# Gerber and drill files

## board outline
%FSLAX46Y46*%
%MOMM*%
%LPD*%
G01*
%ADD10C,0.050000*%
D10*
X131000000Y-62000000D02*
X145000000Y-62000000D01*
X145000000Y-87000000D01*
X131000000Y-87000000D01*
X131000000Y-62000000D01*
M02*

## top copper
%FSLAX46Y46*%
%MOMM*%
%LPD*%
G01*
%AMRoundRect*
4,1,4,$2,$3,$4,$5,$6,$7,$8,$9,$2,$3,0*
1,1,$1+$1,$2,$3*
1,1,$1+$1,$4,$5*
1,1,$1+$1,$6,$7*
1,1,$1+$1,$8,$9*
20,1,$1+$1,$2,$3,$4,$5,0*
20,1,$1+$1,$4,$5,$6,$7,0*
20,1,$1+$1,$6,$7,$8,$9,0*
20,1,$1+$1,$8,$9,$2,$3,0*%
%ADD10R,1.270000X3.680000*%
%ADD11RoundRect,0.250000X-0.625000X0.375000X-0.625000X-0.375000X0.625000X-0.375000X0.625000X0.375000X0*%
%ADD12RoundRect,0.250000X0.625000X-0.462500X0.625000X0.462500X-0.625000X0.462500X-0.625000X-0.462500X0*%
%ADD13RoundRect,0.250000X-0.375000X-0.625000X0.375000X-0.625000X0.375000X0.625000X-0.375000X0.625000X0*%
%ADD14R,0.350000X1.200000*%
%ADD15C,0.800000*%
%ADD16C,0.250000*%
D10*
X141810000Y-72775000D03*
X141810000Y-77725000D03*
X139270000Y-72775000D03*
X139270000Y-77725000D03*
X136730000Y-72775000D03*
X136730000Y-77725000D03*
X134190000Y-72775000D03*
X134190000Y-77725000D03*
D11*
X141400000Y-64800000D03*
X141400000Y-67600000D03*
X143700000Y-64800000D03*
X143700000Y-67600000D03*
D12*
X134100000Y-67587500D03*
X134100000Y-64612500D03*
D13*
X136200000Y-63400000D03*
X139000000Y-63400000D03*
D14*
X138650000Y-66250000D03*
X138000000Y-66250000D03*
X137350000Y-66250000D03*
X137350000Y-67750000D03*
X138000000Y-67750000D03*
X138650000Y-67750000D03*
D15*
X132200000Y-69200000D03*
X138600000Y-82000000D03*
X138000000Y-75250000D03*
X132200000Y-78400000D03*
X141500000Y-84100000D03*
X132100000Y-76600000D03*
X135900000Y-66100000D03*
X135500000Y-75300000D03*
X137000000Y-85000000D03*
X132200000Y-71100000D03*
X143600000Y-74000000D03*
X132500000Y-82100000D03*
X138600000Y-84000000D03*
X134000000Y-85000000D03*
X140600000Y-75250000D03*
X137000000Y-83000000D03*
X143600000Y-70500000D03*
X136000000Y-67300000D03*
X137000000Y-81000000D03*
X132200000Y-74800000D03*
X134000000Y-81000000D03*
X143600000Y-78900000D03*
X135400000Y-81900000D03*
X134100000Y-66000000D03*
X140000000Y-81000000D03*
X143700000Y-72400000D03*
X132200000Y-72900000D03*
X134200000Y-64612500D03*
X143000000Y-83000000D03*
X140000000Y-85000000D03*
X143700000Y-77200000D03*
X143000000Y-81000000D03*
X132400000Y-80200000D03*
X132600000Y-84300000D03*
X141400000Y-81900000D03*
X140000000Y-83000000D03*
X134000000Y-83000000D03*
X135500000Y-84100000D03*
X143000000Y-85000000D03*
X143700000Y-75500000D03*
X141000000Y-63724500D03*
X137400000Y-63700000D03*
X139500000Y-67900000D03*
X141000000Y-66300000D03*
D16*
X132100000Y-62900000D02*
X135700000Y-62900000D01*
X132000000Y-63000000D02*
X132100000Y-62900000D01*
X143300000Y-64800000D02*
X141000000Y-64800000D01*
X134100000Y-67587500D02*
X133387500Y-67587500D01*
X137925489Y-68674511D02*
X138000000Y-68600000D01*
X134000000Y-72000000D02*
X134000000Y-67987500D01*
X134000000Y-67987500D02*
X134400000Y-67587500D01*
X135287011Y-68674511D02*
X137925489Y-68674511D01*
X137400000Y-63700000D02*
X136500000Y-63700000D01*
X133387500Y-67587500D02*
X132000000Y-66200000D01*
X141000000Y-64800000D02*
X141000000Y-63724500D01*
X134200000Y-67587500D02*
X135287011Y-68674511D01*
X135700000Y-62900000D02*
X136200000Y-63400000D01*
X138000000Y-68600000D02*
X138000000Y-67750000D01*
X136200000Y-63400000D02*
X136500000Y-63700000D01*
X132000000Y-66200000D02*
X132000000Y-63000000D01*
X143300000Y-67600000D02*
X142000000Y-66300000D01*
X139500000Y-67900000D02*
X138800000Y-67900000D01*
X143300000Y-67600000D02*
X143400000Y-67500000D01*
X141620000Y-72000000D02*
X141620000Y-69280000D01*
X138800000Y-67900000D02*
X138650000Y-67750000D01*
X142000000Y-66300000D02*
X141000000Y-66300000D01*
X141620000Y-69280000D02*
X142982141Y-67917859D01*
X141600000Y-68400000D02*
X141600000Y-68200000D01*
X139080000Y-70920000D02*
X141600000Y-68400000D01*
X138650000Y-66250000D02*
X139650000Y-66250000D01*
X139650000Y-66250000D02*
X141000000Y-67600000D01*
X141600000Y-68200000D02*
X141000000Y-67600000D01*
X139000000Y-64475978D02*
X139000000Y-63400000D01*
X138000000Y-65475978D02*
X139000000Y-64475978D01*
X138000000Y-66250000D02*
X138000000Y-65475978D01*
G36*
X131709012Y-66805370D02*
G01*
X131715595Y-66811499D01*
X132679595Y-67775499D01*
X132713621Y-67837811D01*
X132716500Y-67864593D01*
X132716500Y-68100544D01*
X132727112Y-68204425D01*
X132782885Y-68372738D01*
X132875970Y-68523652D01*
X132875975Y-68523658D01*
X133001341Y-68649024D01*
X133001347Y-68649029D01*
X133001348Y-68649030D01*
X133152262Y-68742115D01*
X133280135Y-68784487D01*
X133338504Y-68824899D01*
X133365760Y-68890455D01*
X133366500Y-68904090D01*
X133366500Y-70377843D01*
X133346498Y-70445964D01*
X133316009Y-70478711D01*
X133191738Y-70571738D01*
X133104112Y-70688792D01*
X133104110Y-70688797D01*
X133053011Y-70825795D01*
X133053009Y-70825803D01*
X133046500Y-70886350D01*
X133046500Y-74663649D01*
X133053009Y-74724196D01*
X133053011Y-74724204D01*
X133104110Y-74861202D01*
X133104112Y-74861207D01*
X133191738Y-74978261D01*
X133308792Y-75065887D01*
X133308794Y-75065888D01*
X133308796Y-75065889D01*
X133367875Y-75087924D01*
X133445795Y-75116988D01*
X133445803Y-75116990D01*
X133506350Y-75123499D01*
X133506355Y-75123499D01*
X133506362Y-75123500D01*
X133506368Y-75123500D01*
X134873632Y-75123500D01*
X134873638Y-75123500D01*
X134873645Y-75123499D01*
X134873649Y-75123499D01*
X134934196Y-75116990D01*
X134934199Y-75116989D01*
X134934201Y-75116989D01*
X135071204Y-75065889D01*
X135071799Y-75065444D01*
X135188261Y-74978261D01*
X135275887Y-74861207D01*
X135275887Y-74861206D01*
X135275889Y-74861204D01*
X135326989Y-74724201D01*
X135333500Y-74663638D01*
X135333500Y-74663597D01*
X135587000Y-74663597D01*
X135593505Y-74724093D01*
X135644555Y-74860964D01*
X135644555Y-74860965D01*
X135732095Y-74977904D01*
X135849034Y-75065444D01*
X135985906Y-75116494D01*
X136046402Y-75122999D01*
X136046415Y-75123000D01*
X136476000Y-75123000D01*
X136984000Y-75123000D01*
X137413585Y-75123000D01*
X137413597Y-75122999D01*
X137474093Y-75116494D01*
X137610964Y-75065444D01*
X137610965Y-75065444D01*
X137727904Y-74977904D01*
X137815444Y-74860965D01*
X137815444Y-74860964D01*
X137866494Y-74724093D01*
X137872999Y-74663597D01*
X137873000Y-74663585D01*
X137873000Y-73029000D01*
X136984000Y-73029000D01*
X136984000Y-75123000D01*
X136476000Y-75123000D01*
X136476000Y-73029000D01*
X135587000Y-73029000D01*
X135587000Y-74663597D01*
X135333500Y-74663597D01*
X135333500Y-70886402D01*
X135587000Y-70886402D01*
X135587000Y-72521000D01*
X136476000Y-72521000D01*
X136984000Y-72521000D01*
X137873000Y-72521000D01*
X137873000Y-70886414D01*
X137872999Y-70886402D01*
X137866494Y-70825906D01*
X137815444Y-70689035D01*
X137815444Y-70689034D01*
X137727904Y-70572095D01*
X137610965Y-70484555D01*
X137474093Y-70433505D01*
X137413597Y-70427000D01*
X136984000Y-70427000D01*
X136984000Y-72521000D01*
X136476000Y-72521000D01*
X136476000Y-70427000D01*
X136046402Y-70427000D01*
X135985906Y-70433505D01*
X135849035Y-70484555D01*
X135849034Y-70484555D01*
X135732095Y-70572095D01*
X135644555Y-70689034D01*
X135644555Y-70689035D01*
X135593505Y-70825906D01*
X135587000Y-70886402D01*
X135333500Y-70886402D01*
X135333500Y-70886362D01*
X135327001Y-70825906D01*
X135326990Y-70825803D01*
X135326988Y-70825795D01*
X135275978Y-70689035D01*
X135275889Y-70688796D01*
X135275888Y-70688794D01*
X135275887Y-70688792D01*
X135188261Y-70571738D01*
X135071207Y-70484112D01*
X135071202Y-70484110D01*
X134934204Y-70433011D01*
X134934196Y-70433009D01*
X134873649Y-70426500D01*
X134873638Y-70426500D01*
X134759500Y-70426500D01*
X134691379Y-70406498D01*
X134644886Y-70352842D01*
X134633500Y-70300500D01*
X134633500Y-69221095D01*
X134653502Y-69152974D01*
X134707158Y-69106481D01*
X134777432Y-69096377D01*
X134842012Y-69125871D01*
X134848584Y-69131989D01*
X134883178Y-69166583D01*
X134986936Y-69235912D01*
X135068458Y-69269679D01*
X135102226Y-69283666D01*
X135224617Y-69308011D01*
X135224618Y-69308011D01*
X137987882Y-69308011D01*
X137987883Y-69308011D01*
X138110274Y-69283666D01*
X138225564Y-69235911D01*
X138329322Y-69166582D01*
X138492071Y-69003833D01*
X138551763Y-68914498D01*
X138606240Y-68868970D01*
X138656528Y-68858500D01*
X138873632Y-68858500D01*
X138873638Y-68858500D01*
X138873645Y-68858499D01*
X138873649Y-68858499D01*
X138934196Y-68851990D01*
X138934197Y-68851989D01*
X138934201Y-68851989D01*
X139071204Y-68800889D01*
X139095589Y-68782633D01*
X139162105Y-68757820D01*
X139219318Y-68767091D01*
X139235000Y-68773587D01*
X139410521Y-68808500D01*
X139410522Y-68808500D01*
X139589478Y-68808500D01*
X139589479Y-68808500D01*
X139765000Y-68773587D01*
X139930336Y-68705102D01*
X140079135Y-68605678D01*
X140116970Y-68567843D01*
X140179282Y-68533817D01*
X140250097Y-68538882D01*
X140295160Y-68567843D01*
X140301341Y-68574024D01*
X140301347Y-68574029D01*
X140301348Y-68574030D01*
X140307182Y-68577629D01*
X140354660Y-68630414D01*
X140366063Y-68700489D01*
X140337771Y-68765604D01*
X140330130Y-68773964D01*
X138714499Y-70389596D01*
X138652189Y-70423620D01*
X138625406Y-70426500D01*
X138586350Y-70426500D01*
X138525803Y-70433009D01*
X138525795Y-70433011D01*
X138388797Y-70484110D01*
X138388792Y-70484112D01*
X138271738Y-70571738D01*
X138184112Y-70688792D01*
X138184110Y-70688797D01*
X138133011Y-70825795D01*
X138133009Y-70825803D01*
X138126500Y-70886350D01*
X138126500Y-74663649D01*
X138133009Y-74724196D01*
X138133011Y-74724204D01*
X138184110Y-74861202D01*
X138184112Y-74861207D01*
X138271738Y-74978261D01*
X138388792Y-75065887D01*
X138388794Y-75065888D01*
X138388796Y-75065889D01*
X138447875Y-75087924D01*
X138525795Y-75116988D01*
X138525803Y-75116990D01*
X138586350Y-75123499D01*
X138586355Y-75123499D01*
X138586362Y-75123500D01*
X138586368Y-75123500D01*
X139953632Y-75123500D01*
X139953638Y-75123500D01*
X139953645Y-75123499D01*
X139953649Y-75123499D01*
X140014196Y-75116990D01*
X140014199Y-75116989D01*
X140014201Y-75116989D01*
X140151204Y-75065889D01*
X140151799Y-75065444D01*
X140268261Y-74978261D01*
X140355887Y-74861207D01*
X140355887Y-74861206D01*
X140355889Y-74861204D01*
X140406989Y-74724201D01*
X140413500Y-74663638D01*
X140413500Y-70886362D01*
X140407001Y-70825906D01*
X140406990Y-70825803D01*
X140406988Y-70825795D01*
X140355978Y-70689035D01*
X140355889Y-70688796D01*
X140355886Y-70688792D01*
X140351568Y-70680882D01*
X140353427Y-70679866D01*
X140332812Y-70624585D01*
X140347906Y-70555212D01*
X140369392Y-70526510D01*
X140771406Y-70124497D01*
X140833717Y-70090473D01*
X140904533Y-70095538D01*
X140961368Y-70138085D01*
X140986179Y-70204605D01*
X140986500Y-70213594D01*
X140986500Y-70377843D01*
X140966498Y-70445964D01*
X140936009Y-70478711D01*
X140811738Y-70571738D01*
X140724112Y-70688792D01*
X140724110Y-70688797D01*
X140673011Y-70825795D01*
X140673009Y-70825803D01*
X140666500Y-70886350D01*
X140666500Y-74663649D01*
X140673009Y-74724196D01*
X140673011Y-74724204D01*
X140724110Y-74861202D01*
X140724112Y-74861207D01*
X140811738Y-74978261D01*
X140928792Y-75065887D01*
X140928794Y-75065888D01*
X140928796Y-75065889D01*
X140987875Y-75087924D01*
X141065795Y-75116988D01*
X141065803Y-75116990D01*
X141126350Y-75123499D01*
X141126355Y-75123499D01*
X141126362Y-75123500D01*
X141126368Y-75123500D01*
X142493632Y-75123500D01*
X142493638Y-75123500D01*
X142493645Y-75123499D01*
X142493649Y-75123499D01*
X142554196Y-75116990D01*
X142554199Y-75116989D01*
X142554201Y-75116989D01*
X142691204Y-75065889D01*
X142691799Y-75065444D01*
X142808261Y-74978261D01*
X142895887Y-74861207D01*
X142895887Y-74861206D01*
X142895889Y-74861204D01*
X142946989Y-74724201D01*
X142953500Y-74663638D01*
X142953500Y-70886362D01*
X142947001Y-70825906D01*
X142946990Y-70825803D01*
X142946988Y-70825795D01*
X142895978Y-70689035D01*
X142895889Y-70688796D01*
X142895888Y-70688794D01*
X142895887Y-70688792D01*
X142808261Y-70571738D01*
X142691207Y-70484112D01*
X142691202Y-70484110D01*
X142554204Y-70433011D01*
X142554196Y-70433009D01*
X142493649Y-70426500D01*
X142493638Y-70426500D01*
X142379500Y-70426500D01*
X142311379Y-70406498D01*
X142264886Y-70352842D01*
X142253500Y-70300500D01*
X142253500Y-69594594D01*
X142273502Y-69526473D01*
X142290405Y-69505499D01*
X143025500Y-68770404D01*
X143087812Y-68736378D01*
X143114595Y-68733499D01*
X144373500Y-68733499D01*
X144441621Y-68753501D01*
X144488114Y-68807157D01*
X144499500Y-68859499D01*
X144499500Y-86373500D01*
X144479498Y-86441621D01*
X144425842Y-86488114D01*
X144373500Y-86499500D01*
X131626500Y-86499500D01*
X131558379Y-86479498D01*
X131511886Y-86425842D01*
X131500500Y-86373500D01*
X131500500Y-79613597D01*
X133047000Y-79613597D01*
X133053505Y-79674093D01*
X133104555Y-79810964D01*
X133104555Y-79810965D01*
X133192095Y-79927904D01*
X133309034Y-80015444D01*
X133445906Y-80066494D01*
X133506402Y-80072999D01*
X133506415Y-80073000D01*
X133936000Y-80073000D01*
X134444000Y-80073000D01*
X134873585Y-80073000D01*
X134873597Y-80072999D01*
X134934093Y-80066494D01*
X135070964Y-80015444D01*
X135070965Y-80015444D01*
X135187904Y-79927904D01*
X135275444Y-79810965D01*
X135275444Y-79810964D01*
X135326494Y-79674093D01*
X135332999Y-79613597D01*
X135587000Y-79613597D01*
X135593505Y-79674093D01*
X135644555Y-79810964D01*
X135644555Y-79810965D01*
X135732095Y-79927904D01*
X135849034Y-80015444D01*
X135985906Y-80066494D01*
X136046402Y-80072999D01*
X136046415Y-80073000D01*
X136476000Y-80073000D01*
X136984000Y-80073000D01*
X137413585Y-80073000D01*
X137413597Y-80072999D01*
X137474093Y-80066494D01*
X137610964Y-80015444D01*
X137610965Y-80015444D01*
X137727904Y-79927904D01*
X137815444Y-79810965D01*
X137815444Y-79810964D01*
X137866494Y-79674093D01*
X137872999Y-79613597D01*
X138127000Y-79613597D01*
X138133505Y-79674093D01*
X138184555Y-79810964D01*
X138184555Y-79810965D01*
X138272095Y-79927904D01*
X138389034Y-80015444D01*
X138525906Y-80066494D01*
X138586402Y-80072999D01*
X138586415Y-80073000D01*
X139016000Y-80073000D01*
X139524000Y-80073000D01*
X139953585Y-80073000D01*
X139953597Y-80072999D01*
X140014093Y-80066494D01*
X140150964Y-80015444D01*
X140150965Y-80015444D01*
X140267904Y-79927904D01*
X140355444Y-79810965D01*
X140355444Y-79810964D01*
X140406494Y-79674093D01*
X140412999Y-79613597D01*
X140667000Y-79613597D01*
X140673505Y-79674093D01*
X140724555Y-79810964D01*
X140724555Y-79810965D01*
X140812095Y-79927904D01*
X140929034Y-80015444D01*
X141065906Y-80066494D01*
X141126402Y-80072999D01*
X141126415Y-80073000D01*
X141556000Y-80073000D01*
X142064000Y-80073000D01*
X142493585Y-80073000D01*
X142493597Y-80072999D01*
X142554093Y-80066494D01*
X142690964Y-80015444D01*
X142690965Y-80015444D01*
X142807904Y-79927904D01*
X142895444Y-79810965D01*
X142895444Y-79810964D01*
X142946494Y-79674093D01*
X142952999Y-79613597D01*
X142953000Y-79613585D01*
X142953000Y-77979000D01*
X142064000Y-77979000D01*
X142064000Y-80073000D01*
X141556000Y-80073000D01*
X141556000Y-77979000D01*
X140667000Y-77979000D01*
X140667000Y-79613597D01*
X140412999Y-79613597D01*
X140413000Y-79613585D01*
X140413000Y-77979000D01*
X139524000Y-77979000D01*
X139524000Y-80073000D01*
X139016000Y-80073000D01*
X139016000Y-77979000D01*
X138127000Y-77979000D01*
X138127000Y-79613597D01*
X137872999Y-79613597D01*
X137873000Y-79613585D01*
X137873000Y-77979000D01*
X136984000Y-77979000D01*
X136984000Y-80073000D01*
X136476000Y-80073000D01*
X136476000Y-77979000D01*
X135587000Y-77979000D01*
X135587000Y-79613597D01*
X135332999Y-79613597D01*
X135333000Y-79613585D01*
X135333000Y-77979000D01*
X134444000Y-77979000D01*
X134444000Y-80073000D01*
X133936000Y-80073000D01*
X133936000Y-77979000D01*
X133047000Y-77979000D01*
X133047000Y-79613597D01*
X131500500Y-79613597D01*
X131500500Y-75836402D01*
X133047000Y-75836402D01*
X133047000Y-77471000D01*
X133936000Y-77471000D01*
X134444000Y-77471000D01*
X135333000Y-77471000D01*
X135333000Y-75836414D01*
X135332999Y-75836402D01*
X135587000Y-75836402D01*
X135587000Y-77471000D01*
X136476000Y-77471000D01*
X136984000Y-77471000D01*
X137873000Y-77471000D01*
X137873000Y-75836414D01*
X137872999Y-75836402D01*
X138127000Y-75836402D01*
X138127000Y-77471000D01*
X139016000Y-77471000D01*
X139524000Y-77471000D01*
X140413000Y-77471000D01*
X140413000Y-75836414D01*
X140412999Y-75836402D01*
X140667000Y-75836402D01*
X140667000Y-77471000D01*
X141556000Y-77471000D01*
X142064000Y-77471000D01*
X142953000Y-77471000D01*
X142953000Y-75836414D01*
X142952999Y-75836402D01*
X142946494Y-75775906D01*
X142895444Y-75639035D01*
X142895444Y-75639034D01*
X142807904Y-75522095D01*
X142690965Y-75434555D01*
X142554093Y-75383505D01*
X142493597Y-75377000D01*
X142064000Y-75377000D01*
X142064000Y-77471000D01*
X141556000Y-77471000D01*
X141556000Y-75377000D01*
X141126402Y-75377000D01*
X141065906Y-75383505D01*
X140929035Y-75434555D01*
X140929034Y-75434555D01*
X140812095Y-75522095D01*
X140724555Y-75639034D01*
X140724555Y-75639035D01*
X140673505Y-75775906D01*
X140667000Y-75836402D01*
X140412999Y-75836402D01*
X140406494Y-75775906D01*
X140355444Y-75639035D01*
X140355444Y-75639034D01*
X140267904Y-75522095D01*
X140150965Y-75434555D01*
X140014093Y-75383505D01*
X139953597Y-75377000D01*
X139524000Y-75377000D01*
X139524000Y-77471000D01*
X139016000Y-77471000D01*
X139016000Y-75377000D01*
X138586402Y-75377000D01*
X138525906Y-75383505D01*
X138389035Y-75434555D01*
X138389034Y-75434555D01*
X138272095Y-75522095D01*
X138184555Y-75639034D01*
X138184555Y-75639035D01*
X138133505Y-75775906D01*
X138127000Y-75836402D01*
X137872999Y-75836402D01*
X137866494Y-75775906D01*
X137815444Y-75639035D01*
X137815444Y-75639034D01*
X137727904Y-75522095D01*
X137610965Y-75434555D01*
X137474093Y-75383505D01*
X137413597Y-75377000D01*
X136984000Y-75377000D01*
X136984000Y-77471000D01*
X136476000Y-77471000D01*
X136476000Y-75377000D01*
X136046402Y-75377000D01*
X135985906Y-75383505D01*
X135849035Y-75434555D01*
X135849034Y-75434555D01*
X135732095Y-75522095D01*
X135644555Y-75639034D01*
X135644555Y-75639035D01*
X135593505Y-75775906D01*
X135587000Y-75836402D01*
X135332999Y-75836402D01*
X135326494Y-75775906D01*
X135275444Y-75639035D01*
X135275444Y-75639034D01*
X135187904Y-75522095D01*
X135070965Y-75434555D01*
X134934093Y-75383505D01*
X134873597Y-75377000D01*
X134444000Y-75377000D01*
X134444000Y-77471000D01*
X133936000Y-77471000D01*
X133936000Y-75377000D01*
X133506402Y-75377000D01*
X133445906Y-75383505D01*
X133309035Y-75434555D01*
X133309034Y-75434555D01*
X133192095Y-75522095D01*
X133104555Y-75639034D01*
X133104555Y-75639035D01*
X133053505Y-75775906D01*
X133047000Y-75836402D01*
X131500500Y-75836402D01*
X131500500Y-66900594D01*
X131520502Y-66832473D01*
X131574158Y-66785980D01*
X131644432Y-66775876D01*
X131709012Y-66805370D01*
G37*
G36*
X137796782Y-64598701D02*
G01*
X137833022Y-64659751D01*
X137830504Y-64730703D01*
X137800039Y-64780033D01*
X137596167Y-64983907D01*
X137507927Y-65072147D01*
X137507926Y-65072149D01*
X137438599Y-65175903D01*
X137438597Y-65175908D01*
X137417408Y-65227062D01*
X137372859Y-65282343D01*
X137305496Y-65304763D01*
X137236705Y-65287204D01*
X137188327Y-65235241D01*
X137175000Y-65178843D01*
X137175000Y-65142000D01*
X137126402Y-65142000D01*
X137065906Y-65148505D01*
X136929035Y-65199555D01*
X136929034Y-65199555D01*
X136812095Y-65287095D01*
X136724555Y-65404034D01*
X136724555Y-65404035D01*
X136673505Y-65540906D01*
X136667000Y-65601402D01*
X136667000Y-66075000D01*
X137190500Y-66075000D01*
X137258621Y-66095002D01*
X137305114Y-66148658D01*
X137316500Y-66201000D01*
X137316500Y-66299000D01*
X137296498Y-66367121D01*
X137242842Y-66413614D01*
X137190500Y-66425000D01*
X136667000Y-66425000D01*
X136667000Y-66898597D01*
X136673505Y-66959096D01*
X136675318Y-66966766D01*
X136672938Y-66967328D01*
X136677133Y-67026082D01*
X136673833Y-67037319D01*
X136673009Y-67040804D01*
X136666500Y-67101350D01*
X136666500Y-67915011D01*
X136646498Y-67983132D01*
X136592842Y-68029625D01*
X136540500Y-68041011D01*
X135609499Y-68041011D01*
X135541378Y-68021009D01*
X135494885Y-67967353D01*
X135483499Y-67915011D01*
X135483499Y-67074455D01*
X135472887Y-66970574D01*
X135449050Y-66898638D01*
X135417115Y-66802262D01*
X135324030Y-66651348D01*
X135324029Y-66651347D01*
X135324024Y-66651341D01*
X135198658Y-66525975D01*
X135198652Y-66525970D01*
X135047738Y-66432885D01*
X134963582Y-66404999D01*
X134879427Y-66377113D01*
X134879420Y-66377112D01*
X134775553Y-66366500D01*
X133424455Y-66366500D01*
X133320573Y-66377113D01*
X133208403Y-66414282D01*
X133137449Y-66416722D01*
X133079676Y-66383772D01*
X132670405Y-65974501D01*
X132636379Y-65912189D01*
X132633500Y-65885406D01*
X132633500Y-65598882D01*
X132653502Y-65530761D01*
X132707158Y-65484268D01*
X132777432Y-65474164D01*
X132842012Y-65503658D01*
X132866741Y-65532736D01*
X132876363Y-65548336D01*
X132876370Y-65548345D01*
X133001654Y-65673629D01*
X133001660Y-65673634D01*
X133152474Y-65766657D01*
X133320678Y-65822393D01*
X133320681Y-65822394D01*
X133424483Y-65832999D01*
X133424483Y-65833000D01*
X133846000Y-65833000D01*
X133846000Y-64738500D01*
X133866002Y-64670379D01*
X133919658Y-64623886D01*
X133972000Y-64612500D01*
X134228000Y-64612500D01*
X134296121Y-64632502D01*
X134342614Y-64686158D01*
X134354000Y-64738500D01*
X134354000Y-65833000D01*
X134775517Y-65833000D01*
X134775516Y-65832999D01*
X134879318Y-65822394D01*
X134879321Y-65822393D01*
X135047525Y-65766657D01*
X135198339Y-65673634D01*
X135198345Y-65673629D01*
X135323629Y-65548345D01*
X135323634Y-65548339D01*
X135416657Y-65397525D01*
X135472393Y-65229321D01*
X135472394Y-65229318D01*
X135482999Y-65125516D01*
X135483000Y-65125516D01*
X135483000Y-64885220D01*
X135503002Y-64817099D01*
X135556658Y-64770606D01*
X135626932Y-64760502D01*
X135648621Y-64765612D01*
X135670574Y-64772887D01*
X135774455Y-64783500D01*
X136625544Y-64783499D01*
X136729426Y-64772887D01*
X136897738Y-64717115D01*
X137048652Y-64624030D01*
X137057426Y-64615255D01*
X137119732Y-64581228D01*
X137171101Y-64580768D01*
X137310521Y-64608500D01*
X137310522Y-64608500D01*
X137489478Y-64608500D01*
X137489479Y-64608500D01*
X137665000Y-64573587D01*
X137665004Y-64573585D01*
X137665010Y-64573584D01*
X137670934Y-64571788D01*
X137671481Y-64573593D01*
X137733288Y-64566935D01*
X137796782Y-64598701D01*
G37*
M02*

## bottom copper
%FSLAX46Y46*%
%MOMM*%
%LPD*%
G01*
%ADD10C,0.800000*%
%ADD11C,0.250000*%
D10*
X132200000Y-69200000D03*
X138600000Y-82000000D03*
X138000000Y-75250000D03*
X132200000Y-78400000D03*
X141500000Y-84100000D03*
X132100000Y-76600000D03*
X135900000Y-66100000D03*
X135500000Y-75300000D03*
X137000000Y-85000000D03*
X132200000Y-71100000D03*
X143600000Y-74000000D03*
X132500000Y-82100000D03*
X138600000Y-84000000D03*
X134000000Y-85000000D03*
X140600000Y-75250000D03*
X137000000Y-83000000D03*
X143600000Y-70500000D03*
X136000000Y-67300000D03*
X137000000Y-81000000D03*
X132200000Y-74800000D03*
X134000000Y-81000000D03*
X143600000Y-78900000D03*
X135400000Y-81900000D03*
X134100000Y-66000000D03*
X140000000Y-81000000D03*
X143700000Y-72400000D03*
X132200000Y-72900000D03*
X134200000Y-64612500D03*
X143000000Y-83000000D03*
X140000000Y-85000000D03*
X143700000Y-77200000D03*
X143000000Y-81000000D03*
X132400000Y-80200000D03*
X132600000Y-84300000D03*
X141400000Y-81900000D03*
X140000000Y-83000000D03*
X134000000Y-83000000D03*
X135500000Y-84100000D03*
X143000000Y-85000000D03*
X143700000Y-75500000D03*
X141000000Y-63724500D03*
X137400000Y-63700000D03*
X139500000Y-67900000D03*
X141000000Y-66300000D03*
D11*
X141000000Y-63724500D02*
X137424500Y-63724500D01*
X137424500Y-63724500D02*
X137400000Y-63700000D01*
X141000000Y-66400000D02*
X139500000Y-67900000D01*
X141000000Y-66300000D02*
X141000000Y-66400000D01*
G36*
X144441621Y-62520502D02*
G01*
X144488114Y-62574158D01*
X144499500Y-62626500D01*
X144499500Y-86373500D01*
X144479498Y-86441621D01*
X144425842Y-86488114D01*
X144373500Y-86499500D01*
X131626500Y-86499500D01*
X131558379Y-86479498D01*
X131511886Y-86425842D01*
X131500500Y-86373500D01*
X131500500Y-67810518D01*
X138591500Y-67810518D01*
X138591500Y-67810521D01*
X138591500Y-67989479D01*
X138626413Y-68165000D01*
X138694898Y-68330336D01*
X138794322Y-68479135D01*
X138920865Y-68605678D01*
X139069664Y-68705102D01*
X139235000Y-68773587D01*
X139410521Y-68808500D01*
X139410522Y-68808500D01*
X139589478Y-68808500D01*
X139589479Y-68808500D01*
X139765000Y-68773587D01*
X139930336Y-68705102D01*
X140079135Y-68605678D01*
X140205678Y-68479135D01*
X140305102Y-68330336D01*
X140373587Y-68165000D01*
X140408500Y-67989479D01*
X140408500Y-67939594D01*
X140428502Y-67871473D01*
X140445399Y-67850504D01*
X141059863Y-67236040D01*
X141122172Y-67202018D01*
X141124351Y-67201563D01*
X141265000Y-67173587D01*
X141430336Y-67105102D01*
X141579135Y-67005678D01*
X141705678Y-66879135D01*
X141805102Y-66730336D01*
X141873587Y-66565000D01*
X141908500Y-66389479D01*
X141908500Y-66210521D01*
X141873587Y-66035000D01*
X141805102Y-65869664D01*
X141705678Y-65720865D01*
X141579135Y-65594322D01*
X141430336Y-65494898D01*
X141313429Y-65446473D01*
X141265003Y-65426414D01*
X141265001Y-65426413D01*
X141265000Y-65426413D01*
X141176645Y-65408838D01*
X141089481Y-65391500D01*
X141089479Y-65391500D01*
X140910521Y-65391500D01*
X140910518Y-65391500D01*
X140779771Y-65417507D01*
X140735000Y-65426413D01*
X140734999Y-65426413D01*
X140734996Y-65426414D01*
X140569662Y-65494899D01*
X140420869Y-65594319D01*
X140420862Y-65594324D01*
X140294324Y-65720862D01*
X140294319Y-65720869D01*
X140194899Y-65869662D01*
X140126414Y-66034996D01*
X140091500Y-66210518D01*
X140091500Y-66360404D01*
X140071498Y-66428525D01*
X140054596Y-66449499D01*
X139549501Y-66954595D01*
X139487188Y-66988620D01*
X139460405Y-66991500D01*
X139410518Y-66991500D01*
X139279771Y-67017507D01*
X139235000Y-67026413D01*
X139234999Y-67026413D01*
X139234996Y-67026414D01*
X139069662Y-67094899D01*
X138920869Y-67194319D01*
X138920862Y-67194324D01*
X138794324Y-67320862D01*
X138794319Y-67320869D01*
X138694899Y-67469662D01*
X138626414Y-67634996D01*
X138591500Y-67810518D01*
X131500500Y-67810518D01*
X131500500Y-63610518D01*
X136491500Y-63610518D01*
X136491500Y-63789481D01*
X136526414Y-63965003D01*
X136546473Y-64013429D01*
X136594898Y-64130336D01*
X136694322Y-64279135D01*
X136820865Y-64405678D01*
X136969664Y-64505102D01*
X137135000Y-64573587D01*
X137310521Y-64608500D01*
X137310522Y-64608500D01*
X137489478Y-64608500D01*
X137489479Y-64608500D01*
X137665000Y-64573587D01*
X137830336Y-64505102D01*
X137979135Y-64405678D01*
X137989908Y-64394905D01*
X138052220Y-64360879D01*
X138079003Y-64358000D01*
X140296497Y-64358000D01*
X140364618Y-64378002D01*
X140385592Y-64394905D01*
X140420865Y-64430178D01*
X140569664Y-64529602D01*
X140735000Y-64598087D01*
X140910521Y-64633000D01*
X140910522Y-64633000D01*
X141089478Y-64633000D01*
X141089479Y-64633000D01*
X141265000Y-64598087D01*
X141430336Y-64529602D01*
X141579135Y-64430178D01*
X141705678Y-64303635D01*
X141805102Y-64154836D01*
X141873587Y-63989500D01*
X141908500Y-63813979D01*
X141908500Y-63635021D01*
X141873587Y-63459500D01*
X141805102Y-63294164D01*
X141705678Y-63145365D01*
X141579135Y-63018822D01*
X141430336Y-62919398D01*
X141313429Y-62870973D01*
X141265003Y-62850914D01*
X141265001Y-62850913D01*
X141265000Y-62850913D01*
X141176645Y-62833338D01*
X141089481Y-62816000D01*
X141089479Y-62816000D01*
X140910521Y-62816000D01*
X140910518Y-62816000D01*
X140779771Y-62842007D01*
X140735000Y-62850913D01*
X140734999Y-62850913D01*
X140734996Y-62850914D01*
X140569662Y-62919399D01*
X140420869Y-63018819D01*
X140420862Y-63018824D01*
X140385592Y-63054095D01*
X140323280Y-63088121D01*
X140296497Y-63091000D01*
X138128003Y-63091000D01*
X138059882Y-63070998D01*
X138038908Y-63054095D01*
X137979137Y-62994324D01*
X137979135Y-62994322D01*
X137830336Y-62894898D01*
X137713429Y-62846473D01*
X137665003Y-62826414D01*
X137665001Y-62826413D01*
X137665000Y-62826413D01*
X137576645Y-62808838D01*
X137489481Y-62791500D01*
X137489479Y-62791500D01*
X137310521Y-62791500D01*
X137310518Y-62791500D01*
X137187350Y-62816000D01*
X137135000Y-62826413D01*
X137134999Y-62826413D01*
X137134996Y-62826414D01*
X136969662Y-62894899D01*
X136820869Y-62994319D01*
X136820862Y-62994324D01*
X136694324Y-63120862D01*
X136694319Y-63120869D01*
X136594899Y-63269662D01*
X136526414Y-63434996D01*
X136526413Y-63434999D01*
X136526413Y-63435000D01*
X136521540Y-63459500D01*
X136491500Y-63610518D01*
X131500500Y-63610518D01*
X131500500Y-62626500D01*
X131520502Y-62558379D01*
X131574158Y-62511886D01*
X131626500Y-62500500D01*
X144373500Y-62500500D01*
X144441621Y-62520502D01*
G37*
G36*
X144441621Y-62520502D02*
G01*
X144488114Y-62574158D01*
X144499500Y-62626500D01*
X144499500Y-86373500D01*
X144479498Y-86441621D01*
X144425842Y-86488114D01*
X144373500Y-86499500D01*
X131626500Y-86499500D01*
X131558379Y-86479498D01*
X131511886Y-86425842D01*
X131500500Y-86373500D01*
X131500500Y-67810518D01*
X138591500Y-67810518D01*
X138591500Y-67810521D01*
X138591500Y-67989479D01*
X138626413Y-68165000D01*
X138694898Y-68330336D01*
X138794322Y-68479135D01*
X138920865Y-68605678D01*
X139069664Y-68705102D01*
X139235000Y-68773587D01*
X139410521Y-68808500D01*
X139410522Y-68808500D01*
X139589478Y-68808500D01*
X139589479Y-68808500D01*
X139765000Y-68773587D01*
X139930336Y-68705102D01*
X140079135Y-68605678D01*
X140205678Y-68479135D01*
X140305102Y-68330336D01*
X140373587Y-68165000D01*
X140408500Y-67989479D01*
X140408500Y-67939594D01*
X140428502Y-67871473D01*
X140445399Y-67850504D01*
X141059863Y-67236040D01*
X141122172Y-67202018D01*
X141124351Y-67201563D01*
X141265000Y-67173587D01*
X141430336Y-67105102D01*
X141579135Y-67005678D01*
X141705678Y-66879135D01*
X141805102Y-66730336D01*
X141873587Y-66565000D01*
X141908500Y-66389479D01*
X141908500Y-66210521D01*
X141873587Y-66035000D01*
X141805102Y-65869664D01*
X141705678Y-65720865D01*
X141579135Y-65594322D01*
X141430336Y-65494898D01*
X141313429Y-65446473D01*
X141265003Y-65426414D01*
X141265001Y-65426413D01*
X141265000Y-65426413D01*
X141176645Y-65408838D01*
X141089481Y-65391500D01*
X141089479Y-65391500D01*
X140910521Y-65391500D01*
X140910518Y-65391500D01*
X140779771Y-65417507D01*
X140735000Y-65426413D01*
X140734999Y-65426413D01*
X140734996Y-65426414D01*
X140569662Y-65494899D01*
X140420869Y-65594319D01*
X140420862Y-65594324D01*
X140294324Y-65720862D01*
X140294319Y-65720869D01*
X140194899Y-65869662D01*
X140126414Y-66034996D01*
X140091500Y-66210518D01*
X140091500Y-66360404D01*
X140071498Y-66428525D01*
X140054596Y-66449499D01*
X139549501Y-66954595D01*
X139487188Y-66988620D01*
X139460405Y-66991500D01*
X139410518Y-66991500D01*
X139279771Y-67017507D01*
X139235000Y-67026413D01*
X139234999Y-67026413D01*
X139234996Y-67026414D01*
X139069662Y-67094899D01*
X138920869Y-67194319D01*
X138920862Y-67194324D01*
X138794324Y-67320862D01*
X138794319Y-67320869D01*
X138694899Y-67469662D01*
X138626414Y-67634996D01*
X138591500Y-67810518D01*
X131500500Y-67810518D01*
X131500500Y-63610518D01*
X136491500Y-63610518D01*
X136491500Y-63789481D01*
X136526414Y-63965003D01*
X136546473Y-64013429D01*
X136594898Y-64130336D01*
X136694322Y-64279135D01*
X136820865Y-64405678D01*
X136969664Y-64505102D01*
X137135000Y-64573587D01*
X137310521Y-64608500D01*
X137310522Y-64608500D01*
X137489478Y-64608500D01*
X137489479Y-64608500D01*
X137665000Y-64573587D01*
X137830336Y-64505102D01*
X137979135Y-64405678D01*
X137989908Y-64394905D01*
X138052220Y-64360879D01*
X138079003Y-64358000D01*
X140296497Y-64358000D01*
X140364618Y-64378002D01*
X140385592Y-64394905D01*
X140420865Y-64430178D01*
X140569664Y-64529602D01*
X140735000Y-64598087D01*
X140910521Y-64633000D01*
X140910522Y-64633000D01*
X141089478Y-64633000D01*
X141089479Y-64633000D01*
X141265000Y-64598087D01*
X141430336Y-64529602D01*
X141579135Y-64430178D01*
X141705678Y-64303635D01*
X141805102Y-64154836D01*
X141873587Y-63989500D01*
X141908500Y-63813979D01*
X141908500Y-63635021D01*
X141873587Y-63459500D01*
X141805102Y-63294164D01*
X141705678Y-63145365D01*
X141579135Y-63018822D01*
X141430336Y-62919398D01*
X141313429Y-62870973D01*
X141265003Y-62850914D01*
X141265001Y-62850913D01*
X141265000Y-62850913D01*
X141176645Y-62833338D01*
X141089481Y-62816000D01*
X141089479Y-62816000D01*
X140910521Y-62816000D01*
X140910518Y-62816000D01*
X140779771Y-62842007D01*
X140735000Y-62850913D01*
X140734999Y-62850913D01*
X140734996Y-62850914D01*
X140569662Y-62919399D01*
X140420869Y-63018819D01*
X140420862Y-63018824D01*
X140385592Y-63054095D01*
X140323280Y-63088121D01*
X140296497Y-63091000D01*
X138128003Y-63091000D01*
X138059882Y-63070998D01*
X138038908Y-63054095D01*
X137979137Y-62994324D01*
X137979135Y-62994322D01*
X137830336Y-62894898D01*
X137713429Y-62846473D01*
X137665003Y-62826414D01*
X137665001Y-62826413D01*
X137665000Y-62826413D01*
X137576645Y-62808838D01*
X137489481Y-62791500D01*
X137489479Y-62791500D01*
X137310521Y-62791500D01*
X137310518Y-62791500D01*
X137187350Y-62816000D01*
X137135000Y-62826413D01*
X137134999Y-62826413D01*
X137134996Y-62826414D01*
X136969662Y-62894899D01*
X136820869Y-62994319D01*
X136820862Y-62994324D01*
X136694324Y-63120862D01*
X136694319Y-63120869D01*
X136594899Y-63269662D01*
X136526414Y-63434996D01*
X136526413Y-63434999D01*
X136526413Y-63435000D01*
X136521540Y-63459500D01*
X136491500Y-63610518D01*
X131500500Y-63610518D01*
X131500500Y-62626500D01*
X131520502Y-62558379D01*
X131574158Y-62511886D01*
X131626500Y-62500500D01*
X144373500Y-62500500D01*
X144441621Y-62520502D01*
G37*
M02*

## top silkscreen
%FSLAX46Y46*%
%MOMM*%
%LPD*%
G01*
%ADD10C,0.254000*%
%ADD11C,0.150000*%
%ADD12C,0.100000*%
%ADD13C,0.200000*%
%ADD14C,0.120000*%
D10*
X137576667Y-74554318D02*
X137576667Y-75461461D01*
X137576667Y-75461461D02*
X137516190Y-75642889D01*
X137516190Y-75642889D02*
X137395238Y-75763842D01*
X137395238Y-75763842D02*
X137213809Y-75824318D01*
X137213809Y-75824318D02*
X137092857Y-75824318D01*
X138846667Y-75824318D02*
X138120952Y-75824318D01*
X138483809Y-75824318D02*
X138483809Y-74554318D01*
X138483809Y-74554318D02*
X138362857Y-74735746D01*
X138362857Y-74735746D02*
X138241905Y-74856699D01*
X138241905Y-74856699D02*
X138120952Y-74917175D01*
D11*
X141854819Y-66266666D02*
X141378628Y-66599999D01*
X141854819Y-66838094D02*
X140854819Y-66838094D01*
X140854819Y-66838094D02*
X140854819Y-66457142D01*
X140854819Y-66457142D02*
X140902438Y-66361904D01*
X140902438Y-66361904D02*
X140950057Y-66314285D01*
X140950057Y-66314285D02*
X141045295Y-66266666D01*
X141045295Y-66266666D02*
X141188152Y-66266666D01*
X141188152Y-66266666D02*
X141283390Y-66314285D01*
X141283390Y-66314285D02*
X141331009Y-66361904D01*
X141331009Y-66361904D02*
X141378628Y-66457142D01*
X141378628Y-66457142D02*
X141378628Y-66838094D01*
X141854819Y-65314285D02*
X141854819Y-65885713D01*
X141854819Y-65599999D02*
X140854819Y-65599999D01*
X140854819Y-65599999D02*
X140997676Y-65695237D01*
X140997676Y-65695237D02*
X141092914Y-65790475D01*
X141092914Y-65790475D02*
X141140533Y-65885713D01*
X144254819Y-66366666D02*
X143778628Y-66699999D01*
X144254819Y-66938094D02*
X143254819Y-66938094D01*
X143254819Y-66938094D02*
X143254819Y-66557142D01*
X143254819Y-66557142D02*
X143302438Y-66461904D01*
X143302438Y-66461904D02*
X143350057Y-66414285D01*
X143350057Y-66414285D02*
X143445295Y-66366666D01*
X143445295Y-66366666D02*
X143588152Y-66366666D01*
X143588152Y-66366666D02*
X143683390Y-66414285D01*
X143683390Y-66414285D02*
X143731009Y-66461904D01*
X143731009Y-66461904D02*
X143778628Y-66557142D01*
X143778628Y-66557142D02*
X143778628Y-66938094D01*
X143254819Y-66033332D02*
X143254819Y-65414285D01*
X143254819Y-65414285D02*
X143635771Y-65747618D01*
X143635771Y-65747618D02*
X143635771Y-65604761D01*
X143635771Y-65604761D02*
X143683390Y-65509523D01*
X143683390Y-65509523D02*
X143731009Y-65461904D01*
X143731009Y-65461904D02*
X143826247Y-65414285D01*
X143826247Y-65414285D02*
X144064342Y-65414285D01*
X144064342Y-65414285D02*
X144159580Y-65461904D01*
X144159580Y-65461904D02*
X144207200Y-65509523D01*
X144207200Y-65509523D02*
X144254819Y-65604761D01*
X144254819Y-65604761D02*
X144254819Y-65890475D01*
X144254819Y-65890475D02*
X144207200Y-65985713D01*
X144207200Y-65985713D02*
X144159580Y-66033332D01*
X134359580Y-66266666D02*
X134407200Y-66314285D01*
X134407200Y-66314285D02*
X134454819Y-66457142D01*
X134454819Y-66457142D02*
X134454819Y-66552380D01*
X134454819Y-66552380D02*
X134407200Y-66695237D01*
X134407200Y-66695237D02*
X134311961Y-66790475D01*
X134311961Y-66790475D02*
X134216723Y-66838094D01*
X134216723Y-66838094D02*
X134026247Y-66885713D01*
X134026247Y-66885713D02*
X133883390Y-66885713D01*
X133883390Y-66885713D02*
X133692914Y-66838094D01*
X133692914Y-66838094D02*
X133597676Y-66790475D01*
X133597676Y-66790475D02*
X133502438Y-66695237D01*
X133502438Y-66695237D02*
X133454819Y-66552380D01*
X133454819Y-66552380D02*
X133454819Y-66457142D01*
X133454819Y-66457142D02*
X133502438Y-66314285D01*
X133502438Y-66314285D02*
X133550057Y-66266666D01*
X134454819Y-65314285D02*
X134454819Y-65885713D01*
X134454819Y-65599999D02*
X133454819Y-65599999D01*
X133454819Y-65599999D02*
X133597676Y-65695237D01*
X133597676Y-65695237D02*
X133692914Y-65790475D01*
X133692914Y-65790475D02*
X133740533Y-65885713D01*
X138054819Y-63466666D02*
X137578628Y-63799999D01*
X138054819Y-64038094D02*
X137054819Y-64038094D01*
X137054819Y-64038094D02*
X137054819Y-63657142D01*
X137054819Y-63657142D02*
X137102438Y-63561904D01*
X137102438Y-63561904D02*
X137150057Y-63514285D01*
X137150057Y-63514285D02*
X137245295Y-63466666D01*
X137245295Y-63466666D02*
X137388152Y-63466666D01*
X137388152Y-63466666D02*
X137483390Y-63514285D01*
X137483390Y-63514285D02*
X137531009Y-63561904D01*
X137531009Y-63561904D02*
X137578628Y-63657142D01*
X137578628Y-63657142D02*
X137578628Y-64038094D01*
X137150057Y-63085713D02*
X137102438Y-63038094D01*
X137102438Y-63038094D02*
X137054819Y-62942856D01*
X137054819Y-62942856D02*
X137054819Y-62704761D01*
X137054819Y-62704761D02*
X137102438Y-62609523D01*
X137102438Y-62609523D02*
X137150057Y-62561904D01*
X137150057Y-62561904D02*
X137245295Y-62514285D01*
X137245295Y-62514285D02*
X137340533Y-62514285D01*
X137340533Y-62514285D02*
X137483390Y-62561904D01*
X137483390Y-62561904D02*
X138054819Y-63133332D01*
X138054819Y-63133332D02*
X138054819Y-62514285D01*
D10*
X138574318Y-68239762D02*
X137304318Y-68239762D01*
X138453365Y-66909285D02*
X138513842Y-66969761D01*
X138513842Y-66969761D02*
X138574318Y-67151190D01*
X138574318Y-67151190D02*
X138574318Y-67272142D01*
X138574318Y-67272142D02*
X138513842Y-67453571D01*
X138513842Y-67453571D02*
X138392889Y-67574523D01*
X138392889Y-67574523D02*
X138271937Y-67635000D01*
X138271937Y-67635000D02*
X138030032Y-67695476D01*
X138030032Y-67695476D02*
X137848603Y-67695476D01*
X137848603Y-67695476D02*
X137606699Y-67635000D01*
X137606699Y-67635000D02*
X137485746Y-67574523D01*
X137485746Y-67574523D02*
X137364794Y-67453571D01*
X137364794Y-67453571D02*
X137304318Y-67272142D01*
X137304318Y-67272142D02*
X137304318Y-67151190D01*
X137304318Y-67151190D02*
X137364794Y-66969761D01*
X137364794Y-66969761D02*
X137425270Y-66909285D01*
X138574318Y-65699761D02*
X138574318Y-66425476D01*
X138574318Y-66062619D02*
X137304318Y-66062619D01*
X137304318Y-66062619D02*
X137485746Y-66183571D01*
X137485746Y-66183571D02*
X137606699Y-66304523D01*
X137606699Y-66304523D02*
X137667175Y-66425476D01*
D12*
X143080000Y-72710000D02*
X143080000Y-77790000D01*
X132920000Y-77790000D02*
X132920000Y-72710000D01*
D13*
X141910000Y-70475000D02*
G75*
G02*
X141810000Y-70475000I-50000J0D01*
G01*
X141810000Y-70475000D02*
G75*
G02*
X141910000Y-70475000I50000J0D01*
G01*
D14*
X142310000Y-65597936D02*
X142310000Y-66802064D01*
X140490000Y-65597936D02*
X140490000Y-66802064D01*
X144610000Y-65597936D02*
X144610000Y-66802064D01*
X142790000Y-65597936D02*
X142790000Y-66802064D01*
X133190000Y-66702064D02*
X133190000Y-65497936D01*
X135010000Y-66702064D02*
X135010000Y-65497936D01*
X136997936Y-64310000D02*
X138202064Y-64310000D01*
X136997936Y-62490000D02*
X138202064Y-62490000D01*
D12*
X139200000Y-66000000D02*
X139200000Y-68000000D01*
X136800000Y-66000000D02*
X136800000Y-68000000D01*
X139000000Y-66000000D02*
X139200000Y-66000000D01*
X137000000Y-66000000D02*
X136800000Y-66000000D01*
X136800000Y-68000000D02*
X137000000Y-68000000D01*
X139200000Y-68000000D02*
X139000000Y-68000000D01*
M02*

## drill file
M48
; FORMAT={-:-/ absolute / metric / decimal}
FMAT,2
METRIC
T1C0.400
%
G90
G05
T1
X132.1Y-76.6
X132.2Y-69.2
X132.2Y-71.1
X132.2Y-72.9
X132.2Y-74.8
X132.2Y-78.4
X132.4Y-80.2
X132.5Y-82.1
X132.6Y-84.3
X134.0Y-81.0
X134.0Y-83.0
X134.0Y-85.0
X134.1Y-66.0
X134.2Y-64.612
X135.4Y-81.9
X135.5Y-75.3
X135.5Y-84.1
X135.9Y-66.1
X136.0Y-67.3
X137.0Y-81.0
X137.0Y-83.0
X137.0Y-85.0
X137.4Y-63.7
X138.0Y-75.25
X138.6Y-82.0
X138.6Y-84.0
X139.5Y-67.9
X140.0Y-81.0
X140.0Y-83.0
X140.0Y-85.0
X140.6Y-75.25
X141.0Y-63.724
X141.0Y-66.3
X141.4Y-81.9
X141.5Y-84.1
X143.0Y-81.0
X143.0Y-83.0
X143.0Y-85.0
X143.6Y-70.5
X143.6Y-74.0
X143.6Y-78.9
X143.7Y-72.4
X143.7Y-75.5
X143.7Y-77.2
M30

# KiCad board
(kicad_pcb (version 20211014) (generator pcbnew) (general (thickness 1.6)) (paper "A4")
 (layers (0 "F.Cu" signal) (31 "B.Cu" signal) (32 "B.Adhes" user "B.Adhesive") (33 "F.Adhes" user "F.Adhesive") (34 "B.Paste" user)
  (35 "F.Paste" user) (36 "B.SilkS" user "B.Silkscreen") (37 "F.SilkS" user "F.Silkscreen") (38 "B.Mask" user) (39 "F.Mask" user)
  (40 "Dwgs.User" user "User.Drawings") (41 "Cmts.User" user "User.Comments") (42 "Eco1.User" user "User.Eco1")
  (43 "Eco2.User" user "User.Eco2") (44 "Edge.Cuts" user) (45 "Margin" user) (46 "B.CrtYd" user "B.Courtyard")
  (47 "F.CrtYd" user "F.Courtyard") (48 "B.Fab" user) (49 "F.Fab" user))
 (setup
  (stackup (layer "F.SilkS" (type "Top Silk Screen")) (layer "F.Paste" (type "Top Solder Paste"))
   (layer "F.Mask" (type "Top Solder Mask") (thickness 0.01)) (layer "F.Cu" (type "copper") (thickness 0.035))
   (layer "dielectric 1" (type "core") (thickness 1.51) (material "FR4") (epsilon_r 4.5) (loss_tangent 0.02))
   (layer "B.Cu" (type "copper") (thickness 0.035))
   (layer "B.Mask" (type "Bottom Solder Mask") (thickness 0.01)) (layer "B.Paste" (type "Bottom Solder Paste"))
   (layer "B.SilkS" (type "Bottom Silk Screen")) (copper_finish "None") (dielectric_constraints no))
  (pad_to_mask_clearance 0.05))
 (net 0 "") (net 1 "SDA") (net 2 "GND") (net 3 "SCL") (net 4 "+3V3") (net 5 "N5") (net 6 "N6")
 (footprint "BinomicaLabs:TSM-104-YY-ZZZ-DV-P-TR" (layer "F.Cu") (at 138 75.25)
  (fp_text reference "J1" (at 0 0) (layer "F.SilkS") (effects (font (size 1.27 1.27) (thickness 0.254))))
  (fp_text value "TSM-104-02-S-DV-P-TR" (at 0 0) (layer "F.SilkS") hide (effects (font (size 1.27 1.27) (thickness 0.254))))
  (fp_line (start 5.08 -2.54) (end 5.08 2.54) (layer "F.SilkS") (width 0.1))
  (fp_line (start -5.08 2.54) (end -5.08 -2.54) (layer "F.SilkS") (width 0.1))
  (fp_circle (center 3.86 -4.775) (end 3.86 -4.725) (layer "F.SilkS") (width 0.2) (fill none))
  (pad "1" smd rect locked (at 3.81 -2.475) (size 1.27 3.68) (layers "F.Cu" "F.Paste" "F.Mask") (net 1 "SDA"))
  (pad "2" smd rect locked (at 3.81 2.475) (size 1.27 3.68) (layers "F.Cu" "F.Paste" "F.Mask") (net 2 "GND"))
  (pad "3" smd rect locked (at 1.27 -2.475) (size 1.27 3.68) (layers "F.Cu" "F.Paste" "F.Mask") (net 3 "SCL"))
  (pad "4" smd rect locked (at 1.27 2.475) (size 1.27 3.68) (layers "F.Cu" "F.Paste" "F.Mask") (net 2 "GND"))
  (pad "5" smd rect locked (at -1.27 -2.475) (size 1.27 3.68) (layers "F.Cu" "F.Paste" "F.Mask") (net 2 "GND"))
  (pad "6" smd rect locked (at -1.27 2.475) (size 1.27 3.68) (layers "F.Cu" "F.Paste" "F.Mask") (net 2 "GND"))
  (pad "7" smd rect locked (at -3.81 -2.475) (size 1.27 3.68) (layers "F.Cu" "F.Paste" "F.Mask") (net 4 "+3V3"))
  (pad "8" smd rect locked (at -3.81 2.475) (size 1.27 3.68) (layers "F.Cu" "F.Paste" "F.Mask") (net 2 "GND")))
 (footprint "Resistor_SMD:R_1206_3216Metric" (layer "F.Cu") (at 141.4 66.2 -90)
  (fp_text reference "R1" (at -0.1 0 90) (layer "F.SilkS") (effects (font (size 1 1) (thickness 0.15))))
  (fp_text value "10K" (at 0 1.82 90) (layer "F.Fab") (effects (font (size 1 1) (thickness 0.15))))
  (fp_line (start -0.602064 -0.91) (end 0.602064 -0.91) (layer "F.SilkS") (width 0.12))
  (fp_line (start -0.602064 0.91) (end 0.602064 0.91) (layer "F.SilkS") (width 0.12))
  (pad "1" smd roundrect locked (at -1.4 0 270) (size 1.25 1.75) (layers "F.Cu" "F.Paste" "F.Mask") (roundrect_rratio 0.2) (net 4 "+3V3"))
  (pad "2" smd roundrect locked (at 1.4 0 270) (size 1.25 1.75) (layers "F.Cu" "F.Paste" "F.Mask") (roundrect_rratio 0.2) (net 3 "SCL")))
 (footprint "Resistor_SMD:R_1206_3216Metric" (layer "F.Cu") (at 143.7 66.2 -90)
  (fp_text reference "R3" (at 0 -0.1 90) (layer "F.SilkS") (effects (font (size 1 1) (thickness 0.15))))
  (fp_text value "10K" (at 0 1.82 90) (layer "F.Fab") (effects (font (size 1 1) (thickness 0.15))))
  (fp_line (start -0.602064 -0.91) (end 0.602064 -0.91) (layer "F.SilkS") (width 0.12))
  (fp_line (start -0.602064 0.91) (end 0.602064 0.91) (layer "F.SilkS") (width 0.12))
  (pad "1" smd roundrect locked (at -1.4 0 270) (size 1.25 1.75) (layers "F.Cu" "F.Paste" "F.Mask") (roundrect_rratio 0.2) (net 4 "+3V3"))
  (pad "2" smd roundrect locked (at 1.4 0 270) (size 1.25 1.75) (layers "F.Cu" "F.Paste" "F.Mask") (roundrect_rratio 0.2) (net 1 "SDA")))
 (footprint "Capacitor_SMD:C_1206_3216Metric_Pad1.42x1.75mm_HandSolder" (layer "F.Cu") (at 134.1 66.1 90)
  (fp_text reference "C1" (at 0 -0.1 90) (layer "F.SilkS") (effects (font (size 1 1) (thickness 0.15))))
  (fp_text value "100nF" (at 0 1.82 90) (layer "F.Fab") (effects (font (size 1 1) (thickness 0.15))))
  (fp_line (start -0.602064 -0.91) (end 0.602064 -0.91) (layer "F.SilkS") (width 0.12))
  (fp_line (start -0.602064 0.91) (end 0.602064 0.91) (layer "F.SilkS") (width 0.12))
  (pad "1" smd roundrect locked (at -1.4875 0 90) (size 1.425 1.75) (layers "F.Cu" "F.Paste" "F.Mask") (roundrect_rratio 0.1754385965)
   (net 4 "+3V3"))
  (pad "2" smd roundrect locked (at 1.4875 0 90) (size 1.425 1.75) (layers "F.Cu" "F.Paste" "F.Mask") (roundrect_rratio 0.1754385965)
   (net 2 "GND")))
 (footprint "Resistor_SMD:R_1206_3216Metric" (layer "F.Cu") (at 137.6 63.4)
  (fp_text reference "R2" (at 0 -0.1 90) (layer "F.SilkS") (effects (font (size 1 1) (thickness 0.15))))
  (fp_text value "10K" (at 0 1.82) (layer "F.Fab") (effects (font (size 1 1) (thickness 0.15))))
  (fp_line (start -0.602064 0.91) (end 0.602064 0.91) (layer "F.SilkS") (width 0.12))
  (fp_line (start -0.602064 -0.91) (end 0.602064 -0.91) (layer "F.SilkS") (width 0.12))
  (pad "1" smd roundrect locked (at -1.4 0) (size 1.25 1.75) (layers "F.Cu" "F.Paste" "F.Mask") (roundrect_rratio 0.2) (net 4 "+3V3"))
  (pad "2" smd roundrect locked (at 1.4 0) (size 1.25 1.75) (layers "F.Cu" "F.Paste" "F.Mask") (roundrect_rratio 0.2) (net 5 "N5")))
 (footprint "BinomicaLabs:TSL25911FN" (layer "F.Cu") (at 138 67 -90)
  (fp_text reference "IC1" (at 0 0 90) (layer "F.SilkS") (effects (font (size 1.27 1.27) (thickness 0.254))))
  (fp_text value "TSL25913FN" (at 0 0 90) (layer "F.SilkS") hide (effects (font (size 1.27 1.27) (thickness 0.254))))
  (fp_line (start -1 -1.2) (end 1 -1.2) (layer "F.SilkS") (width 0.1))
  (fp_line (start -1 1.2) (end 1 1.2) (layer "F.SilkS") (width 0.1))
  (fp_line (start -1 -1) (end -1 -1.2) (layer "F.SilkS") (width 0.1))
  (fp_line (start -1 1) (end -1 1.2) (layer "F.SilkS") (width 0.1))
  (fp_line (start 1 1.2) (end 1 1) (layer "F.SilkS") (width 0.1))
  (fp_line (start 1 -1.2) (end 1 -1) (layer "F.SilkS") (width 0.1))
  (pad "1" smd rect locked (at -0.75 -0.65) (size 0.35 1.2) (layers "F.Cu" "F.Paste" "F.Mask") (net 3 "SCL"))
  (pad "2" smd rect locked (at -0.75 0) (size 0.35 1.2) (layers "F.Cu" "F.Paste" "F.Mask") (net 5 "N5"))
  (pad "3" smd rect locked (at -0.75 0.65) (size 0.35 1.2) (layers "F.Cu" "F.Paste" "F.Mask") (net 2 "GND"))
  (pad "4" smd rect locked (at 0.75 0.65) (size 0.35 1.2) (layers "F.Cu" "F.Paste" "F.Mask") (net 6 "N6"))
  (pad "5" smd rect locked (at 0.75 0) (size 0.35 1.2) (layers "F.Cu" "F.Paste" "F.Mask") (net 4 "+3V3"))
  (pad "6" smd rect locked (at 0.75 -0.65) (size 0.35 1.2) (layers "F.Cu" "F.Paste" "F.Mask") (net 1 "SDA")))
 (gr_rect (start 131 62) (end 145 87) (layer "Edge.Cuts") (width 0.05) (fill none))
 (via (at 132.2 69.2) (size 0.8) (drill 0.4) (layers "F.Cu" "B.Cu") (free) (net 2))
 (via (at 138.6 82) (size 0.8) (drill 0.4) (layers "F.Cu" "B.Cu") (free) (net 2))
 (via (at 138 75.25) (size 0.8) (drill 0.4) (layers "F.Cu" "B.Cu") (free) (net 2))
 (via (at 132.2 78.4) (size 0.8) (drill 0.4) (layers "F.Cu" "B.Cu") (free) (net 2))
 (via (at 141.5 84.1) (size 0.8) (drill 0.4) (layers "F.Cu" "B.Cu") (free) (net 2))
 (via (at 132.1 76.6) (size 0.8) (drill 0.4) (layers "F.Cu" "B.Cu") (free) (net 2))
 (via (at 135.9 66.1) (size 0.8) (drill 0.4) (layers "F.Cu" "B.Cu") (free) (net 2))
 (via (at 135.5 75.3) (size 0.8) (drill 0.4) (layers "F.Cu" "B.Cu") (free) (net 2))
 (via (at 137 85) (size 0.8) (drill 0.4) (layers "F.Cu" "B.Cu") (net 2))
 (via (at 132.2 71.1) (size 0.8) (drill 0.4) (layers "F.Cu" "B.Cu") (free) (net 2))
 (via (at 143.6 74) (size 0.8) (drill 0.4) (layers "F.Cu" "B.Cu") (free) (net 2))
 (via (at 132.5 82.1) (size 0.8) (drill 0.4) (layers "F.Cu" "B.Cu") (free) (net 2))
 (via (at 138.6 84) (size 0.8) (drill 0.4) (layers "F.Cu" "B.Cu") (free) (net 2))
 (via (at 134 85) (size 0.8) (drill 0.4) (layers "F.Cu" "B.Cu") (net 2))
 (via (at 140.6 75.25) (size 0.8) (drill 0.4) (layers "F.Cu" "B.Cu") (free) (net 2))
 (via (at 137 83) (size 0.8) (drill 0.4) (layers "F.Cu" "B.Cu") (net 2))
 (via (at 143.6 70.5) (size 0.8) (drill 0.4) (layers "F.Cu" "B.Cu") (free) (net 2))
 (via (at 136 67.3) (size 0.8) (drill 0.4) (layers "F.Cu" "B.Cu") (free) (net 2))
 (via (at 137 81) (size 0.8) (drill 0.4) (layers "F.Cu" "B.Cu") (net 2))
 (via (at 132.2 74.8) (size 0.8) (drill 0.4) (layers "F.Cu" "B.Cu") (free) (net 2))
 (via (at 134 81) (size 0.8) (drill 0.4) (layers "F.Cu" "B.Cu") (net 2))
 (via (at 143.6 78.9) (size 0.8) (drill 0.4) (layers "F.Cu" "B.Cu") (free) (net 2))
 (via (at 135.4 81.9) (size 0.8) (drill 0.4) (layers "F.Cu" "B.Cu") (free) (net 2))
 (via (at 134.1 66) (size 0.8) (drill 0.4) (layers "F.Cu" "B.Cu") (free) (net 2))
 (via (at 140 81) (size 0.8) (drill 0.4) (layers "F.Cu" "B.Cu") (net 2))
 (via (at 143.7 72.4) (size 0.8) (drill 0.4) (layers "F.Cu" "B.Cu") (free) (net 2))
 (via (at 132.2 72.9) (size 0.8) (drill 0.4) (layers "F.Cu" "B.Cu") (free) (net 2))
 (via (at 134.2 64.6125) (size 0.8) (drill 0.4) (layers "F.Cu" "B.Cu") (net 2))
 (via (at 143 83) (size 0.8) (drill 0.4) (layers "F.Cu" "B.Cu") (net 2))
 (via (at 140 85) (size 0.8) (drill 0.4) (layers "F.Cu" "B.Cu") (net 2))
 (via (at 143.7 77.2) (size 0.8) (drill 0.4) (layers "F.Cu" "B.Cu") (free) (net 2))
 (via (at 143 81) (size 0.8) (drill 0.4) (layers "F.Cu" "B.Cu") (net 2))
 (via (at 132.4 80.2) (size 0.8) (drill 0.4) (layers "F.Cu" "B.Cu") (free) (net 2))
 (via (at 132.6 84.3) (size 0.8) (drill 0.4) (layers "F.Cu" "B.Cu") (free) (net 2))
 (via (at 141.4 81.9) (size 0.8) (drill 0.4) (layers "F.Cu" "B.Cu") (free) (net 2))
 (via (at 140 83) (size 0.8) (drill 0.4) (layers "F.Cu" "B.Cu") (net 2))
 (via (at 134 83) (size 0.8) (drill 0.4) (layers "F.Cu" "B.Cu") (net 2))
 (via (at 135.5 84.1) (size 0.8) (drill 0.4) (layers "F.Cu" "B.Cu") (free) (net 2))
 (via (at 143 85) (size 0.8) (drill 0.4) (layers "F.Cu" "B.Cu") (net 2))
 (via (at 143.7 75.5) (size 0.8) (drill 0.4) (layers "F.Cu" "B.Cu") (free) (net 2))
 (segment (start 132.1 62.9) (end 135.7 62.9) (width 0.25) (layer "F.Cu") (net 4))
 (segment (start 132 63) (end 132.1 62.9) (width 0.25) (layer "F.Cu") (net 4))
 (segment (start 143.3 64.8) (end 141 64.8) (width 0.25) (layer "F.Cu") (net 4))
 (segment (start 134.1 67.5875) (end 133.3875 67.5875) (width 0.25) (layer "F.Cu") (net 4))
 (segment (start 137.925489 68.674511) (end 138 68.6) (width 0.25) (layer "F.Cu") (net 4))
 (segment (start 134 72) (end 134 67.9875) (width 0.25) (layer "F.Cu") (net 4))
 (segment (start 134 67.9875) (end 134.4 67.5875) (width 0.25) (layer "F.Cu") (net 4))
 (segment (start 135.287011 68.674511) (end 137.925489 68.674511) (width 0.25) (layer "F.Cu") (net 4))
 (segment (start 137.4 63.7) (end 136.5 63.7) (width 0.25) (layer "F.Cu") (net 4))
 (segment (start 133.3875 67.5875) (end 132 66.2) (width 0.25) (layer "F.Cu") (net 4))
 (segment (start 141 64.8) (end 141 63.7245) (width 0.25) (layer "F.Cu") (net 4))
 (segment (start 134.2 67.5875) (end 135.287011 68.674511) (width 0.25) (layer "F.Cu") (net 4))
 (segment (start 135.7 62.9) (end 136.2 63.4) (width 0.25) (layer "F.Cu") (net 4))
 (segment (start 138 68.6) (end 138 67.75) (width 0.25) (layer "F.Cu") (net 4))
 (segment (start 136.2 63.4) (end 136.5 63.7) (width 0.25) (layer "F.Cu") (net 4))
 (segment (start 132 66.2) (end 132 63) (width 0.25) (layer "F.Cu") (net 4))
 (via (at 141 63.7245) (size 0.8) (drill 0.4) (layers "F.Cu" "B.Cu") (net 4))
 (via (at 137.4 63.7) (size 0.8) (drill 0.4) (layers "F.Cu" "B.Cu") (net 4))
 (segment (start 141 63.7245) (end 137.4245 63.7245) (width 0.25) (layer "B.Cu") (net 4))
 (segment (start 137.4245 63.7245) (end 137.4 63.7) (width 0.25) (layer "B.Cu") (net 4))
 (segment (start 143.3 67.6) (end 142 66.3) (width 0.25) (layer "F.Cu") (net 1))
 (segment (start 139.5 67.9) (end 138.8 67.9) (width 0.25) (layer "F.Cu") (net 1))
 (segment (start 143.3 67.6) (end 143.4 67.5) (width 0.25) (layer "F.Cu") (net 1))
 (segment (start 141.62 72) (end 141.62 69.28) (width 0.25) (layer "F.Cu") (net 1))
 (segment (start 138.8 67.9) (end 138.65 67.75) (width 0.25) (layer "F.Cu") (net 1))
 (segment (start 142 66.3) (end 141 66.3) (width 0.25) (layer "F.Cu") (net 1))
 (segment (start 141.62 69.28) (end 142.982141 67.917859) (width 0.25) (layer "F.Cu") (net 1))
 (via (at 139.5 67.9) (size 0.8) (drill 0.4) (layers "F.Cu" "B.Cu") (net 1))
 (via (at 141 66.3) (size 0.8) (drill 0.4) (layers "F.Cu" "B.Cu") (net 1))
 (segment (start 141 66.4) (end 139.5 67.9) (width 0.25) (layer "B.Cu") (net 1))
 (segment (start 141 66.3) (end 141 66.4) (width 0.25) (layer "B.Cu") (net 1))
 (segment (start 141.6 68.4) (end 141.6 68.2) (width 0.25) (layer "F.Cu") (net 3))
 (segment (start 139.08 70.92) (end 141.6 68.4) (width 0.25) (layer "F.Cu") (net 3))
 (segment (start 138.65 66.25) (end 139.65 66.25) (width 0.25) (layer "F.Cu") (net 3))
 (segment (start 139.65 66.25) (end 141 67.6) (width 0.25) (layer "F.Cu") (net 3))
 (segment (start 141.6 68.2) (end 141 67.6) (width 0.25) (layer "F.Cu") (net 3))
 (segment (start 139 64.475978) (end 139 63.4) (width 0.25) (layer "F.Cu") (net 5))
 (segment (start 138 65.475978) (end 139 64.475978) (width 0.25) (layer "F.Cu") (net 5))
 (segment (start 138 66.25) (end 138 65.475978) (width 0.25) (layer "F.Cu") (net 5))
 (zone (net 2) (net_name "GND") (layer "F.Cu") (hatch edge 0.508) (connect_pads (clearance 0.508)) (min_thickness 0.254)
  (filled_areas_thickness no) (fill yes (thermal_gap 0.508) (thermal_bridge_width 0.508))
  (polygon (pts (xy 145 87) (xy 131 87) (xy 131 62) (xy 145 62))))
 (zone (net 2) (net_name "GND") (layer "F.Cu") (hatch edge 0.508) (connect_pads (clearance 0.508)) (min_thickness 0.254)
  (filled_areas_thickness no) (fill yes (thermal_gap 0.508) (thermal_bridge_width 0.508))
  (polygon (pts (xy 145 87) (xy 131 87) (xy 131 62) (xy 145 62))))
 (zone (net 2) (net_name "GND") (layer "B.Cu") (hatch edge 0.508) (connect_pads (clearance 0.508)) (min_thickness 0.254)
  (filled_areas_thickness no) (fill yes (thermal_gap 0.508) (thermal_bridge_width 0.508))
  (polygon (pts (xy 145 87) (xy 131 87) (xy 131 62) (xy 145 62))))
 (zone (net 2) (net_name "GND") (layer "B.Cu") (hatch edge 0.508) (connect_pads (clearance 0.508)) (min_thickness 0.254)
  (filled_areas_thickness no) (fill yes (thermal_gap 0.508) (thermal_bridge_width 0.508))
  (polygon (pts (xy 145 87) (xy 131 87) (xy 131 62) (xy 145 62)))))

